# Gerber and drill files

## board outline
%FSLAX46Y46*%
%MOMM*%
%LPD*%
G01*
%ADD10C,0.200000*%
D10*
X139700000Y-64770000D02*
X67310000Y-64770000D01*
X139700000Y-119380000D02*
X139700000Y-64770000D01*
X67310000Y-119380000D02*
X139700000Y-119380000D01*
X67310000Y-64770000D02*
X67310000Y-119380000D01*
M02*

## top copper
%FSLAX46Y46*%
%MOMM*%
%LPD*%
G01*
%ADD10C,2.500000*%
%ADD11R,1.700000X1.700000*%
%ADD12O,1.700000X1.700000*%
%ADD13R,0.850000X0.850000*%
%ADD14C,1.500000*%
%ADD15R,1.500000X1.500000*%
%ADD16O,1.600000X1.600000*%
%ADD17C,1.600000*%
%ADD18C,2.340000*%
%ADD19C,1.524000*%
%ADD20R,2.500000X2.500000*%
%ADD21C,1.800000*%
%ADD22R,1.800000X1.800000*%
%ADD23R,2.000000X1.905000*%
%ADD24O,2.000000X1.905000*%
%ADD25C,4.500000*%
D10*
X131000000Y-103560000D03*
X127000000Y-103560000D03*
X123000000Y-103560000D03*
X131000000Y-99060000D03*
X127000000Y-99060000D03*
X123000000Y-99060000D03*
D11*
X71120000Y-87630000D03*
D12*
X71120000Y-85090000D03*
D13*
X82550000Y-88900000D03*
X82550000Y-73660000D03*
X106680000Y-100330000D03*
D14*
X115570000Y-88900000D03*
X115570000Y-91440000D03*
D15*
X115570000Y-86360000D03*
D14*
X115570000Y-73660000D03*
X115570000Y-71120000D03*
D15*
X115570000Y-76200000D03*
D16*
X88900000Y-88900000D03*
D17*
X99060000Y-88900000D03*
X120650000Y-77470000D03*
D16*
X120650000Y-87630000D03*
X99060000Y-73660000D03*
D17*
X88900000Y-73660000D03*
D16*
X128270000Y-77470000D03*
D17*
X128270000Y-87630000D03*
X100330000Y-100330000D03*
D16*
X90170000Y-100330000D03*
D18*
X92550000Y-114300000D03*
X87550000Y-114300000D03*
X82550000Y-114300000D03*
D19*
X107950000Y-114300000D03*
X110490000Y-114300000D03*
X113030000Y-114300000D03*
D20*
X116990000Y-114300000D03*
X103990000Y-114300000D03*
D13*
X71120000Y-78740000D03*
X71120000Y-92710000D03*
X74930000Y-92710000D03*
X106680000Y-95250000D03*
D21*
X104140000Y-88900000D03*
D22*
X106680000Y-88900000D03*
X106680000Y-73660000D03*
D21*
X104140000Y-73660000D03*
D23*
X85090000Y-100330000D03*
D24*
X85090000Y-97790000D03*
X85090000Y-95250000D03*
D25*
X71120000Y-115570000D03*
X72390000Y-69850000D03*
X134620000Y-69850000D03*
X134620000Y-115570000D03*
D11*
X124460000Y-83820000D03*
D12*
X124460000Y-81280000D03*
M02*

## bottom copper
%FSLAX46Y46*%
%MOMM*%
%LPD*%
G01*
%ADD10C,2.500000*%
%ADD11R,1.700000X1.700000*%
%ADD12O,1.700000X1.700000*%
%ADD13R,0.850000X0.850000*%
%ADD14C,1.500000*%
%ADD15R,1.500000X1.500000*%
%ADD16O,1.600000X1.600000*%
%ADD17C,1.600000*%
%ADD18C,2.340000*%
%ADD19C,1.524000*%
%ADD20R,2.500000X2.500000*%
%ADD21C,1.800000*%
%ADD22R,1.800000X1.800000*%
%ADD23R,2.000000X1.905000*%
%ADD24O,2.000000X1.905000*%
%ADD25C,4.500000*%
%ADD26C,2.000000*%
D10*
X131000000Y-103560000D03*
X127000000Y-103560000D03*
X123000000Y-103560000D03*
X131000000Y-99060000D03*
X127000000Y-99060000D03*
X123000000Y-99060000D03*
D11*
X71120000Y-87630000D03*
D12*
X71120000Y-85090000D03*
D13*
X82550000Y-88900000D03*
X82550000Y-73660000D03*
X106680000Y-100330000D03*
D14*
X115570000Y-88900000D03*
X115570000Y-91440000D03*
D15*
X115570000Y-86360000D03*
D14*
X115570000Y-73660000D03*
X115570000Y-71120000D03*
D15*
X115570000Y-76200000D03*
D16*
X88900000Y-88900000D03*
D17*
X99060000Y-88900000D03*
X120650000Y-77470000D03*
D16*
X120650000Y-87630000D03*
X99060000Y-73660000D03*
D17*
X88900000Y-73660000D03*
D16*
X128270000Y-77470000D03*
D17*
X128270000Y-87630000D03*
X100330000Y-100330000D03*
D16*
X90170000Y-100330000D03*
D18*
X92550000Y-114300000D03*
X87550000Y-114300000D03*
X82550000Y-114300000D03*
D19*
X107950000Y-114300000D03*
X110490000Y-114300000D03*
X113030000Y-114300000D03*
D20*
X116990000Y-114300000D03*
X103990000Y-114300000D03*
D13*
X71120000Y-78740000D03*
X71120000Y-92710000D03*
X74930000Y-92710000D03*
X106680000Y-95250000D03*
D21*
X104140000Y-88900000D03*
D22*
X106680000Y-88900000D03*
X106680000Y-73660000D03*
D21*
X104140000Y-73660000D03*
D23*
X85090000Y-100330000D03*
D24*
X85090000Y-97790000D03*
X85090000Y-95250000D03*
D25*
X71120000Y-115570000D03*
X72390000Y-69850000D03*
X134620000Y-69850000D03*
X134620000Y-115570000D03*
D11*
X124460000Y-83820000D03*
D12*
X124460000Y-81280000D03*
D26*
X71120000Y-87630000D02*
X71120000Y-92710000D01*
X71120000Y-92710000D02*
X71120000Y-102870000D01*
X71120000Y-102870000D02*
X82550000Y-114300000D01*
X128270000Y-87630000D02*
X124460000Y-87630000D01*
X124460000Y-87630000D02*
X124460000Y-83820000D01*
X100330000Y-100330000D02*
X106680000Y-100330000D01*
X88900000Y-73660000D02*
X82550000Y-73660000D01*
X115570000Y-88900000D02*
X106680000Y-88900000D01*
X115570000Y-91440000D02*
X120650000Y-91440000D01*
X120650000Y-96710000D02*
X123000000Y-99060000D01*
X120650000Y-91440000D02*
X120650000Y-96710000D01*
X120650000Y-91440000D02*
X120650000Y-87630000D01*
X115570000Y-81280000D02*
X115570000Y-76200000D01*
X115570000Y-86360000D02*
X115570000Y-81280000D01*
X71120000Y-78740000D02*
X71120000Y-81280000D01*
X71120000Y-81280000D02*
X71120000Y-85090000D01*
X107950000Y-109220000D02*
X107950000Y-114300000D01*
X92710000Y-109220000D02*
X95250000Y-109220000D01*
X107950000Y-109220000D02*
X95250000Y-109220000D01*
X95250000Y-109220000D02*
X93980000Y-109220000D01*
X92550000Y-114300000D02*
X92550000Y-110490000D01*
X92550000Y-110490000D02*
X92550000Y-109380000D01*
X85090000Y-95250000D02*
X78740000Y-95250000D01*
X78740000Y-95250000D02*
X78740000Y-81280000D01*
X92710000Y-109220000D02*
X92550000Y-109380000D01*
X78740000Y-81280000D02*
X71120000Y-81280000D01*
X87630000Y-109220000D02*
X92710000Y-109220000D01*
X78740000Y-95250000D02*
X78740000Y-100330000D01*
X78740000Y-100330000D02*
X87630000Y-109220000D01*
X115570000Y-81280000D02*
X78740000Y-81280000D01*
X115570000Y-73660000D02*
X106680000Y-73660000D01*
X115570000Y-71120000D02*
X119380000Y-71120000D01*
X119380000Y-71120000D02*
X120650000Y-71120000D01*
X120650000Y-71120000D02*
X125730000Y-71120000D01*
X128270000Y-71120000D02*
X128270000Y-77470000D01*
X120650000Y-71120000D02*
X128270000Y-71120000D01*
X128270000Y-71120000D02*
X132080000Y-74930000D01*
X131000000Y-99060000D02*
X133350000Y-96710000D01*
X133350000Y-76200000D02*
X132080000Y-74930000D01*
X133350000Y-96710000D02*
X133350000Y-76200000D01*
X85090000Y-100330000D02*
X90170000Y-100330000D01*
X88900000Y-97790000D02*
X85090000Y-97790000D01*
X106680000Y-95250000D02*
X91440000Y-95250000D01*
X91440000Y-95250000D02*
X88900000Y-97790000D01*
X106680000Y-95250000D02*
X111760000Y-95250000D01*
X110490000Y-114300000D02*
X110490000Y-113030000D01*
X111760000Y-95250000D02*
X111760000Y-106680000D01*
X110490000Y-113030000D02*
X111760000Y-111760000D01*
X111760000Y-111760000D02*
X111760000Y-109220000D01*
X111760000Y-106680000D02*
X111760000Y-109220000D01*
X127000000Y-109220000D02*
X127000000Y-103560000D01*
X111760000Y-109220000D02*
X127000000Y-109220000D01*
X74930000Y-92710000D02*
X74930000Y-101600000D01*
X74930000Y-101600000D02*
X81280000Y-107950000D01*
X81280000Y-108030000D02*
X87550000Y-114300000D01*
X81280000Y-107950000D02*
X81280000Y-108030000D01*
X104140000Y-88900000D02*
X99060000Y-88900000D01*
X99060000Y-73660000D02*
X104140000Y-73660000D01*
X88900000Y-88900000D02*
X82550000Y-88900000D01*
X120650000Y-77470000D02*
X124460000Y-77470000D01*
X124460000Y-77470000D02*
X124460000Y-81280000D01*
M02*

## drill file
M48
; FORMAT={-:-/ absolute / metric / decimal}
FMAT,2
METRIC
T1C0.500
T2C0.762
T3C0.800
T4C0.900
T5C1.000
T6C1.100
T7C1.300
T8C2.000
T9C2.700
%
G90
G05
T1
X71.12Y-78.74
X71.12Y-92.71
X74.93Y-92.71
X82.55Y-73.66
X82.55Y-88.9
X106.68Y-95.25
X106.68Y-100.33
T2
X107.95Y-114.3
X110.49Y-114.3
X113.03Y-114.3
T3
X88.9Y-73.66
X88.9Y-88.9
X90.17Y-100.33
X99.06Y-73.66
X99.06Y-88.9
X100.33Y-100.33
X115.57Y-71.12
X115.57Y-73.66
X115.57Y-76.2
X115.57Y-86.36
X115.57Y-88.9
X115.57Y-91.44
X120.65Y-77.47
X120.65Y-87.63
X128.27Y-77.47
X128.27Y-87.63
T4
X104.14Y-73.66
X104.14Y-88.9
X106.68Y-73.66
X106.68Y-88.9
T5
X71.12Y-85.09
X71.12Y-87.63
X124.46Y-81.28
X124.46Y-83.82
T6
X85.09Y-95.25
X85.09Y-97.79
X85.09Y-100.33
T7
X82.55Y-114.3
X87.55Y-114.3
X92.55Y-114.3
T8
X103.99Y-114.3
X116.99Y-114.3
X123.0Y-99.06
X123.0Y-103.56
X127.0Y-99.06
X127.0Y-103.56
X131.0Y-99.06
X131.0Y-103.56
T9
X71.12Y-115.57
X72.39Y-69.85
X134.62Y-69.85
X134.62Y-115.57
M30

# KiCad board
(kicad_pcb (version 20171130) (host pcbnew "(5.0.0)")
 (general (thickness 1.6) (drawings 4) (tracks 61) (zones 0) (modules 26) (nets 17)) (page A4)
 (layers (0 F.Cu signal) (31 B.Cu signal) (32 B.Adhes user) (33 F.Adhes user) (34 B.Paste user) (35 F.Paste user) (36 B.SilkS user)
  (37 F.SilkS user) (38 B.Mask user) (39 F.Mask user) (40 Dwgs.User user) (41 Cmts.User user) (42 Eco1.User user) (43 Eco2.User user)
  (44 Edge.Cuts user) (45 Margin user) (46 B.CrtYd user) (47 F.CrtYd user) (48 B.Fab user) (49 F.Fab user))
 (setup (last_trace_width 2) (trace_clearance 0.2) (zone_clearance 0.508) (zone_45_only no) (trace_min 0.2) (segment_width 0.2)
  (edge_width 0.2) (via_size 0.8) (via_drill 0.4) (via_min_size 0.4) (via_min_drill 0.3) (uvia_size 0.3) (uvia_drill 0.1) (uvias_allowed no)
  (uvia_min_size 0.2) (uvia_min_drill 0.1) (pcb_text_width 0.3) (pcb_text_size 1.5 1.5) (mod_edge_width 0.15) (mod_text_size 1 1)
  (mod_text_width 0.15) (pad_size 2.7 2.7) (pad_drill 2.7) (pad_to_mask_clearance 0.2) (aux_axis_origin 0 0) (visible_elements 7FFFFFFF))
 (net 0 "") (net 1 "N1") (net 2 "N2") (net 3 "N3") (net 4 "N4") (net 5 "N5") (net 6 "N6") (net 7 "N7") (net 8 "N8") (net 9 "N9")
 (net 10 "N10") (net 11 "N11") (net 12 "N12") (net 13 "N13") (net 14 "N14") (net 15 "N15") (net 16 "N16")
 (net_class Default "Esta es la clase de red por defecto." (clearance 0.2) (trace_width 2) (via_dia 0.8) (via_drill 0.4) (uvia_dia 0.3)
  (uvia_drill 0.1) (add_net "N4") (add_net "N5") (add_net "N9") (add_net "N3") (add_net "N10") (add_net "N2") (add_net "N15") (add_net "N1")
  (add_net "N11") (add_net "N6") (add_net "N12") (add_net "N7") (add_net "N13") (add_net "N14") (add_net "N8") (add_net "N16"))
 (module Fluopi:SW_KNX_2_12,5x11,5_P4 (layer F.Cu) (at 127 99.06)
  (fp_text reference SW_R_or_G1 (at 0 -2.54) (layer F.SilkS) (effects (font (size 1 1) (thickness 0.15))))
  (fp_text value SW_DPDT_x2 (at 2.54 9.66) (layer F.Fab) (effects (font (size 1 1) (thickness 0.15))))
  (pad 6 thru_hole circle (at 4 4.5) (size 2.5 2.5) (drill 2) (layers *.Cu *.Mask))
  (pad 2 thru_hole circle (at 0 4.5) (size 2.5 2.5) (drill 2) (layers *.Cu *.Mask) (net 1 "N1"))
  (pad 4 thru_hole circle (at -4 4.5) (size 2.5 2.5) (drill 2) (layers *.Cu *.Mask))
  (pad 3 thru_hole circle (at 4 0) (size 2.5 2.5) (drill 2) (layers *.Cu *.Mask) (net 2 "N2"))
  (pad 5 thru_hole circle (at 0 0) (size 2.5 2.5) (drill 2) (layers *.Cu *.Mask))
  (pad 1 thru_hole circle (at -4 0) (size 2.5 2.5) (drill 2) (layers *.Cu *.Mask) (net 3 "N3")))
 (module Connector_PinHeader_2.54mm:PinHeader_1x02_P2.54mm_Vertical (layer F.Cu) (at 71.12 87.63 180)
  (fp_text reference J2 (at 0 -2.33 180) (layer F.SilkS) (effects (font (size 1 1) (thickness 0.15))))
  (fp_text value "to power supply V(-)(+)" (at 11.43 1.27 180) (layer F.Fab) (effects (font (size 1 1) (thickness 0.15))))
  (pad 1 thru_hole rect (at 0 0 180) (size 1.7 1.7) (drill 1) (layers *.Cu *.Mask) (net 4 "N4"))
  (pad 2 thru_hole oval (at 0 2.54 180) (size 1.7 1.7) (drill 1) (layers *.Cu *.Mask) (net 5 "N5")))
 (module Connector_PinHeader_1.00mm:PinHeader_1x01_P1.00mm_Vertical (layer F.Cu) (at 82.55 88.9)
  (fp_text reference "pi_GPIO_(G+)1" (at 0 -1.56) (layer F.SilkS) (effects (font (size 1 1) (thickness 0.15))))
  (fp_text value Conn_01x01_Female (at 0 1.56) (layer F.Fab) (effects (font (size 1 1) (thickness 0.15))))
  (pad 1 thru_hole rect (at 0 0) (size 0.85 0.85) (drill 0.5) (layers *.Cu *.Mask) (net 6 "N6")))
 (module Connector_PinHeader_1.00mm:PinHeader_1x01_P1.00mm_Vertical (layer F.Cu) (at 82.55 73.66 180)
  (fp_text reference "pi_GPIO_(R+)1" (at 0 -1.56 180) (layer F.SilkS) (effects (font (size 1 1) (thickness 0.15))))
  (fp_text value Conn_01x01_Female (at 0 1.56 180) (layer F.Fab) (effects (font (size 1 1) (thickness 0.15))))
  (pad 1 thru_hole rect (at 0 0 180) (size 0.85 0.85) (drill 0.5) (layers *.Cu *.Mask) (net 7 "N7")))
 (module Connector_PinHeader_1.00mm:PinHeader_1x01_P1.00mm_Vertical (layer F.Cu) (at 106.68 100.33)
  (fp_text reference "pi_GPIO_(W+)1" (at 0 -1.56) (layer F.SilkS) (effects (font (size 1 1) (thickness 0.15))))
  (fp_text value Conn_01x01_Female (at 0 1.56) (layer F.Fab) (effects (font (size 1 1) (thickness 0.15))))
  (pad 1 thru_hole rect (at 0 0) (size 0.85 0.85) (drill 0.5) (layers *.Cu *.Mask) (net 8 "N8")))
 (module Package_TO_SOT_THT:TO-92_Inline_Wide (layer F.Cu) (at 115.57 86.36 270)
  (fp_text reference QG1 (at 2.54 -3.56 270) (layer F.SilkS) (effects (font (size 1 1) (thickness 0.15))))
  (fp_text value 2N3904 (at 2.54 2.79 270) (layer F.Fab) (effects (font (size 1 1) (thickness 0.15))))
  (pad 2 thru_hole circle (at 2.54 0) (size 1.5 1.5) (drill 0.8) (layers *.Cu *.Mask) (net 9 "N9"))
  (pad 3 thru_hole circle (at 5.08 0) (size 1.5 1.5) (drill 0.8) (layers *.Cu *.Mask) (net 3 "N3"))
  (pad 1 thru_hole rect (at 0 0) (size 1.5 1.5) (drill 0.8) (layers *.Cu *.Mask) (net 5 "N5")))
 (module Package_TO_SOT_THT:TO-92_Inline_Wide (layer F.Cu) (at 115.57 76.2 90)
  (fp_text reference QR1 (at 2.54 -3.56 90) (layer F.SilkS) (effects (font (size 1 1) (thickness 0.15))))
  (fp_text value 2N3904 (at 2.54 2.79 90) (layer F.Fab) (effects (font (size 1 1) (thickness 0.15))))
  (pad 2 thru_hole circle (at 2.54 0 180) (size 1.5 1.5) (drill 0.8) (layers *.Cu *.Mask) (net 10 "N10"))
  (pad 3 thru_hole circle (at 5.08 0 180) (size 1.5 1.5) (drill 0.8) (layers *.Cu *.Mask) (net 2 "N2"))
  (pad 1 thru_hole rect (at 0 0 180) (size 1.5 1.5) (drill 0.8) (layers *.Cu *.Mask) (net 5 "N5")))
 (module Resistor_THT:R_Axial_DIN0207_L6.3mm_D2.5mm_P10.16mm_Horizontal (layer F.Cu) (at 99.06 88.9 180)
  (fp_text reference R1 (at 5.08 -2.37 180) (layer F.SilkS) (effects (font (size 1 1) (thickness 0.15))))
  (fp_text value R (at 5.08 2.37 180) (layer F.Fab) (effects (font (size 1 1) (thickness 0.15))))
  (pad 2 thru_hole oval (at 10.16 0 180) (size 1.6 1.6) (drill 0.8) (layers *.Cu *.Mask) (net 6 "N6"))
  (pad 1 thru_hole circle (at 0 0 180) (size 1.6 1.6) (drill 0.8) (layers *.Cu *.Mask) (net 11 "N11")))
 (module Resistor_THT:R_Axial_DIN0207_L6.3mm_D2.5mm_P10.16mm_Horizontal (layer F.Cu) (at 120.65 77.47 270)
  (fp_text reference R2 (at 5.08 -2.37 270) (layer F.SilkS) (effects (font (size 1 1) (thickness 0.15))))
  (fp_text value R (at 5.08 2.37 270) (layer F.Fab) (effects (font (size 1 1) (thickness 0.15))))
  (pad 1 thru_hole circle (at 0 0 270) (size 1.6 1.6) (drill 0.8) (layers *.Cu *.Mask) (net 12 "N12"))
  (pad 2 thru_hole oval (at 10.16 0 270) (size 1.6 1.6) (drill 0.8) (layers *.Cu *.Mask) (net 3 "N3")))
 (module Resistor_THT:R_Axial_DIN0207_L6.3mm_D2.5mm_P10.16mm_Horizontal (layer F.Cu) (at 88.9 73.66)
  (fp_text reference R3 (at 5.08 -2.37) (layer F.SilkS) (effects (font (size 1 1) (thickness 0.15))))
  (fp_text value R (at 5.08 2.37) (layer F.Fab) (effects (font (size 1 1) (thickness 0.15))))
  (pad 2 thru_hole oval (at 10.16 0) (size 1.6 1.6) (drill 0.8) (layers *.Cu *.Mask) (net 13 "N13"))
  (pad 1 thru_hole circle (at 0 0) (size 1.6 1.6) (drill 0.8) (layers *.Cu *.Mask) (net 7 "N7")))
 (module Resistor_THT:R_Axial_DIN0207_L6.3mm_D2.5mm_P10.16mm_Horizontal (layer F.Cu) (at 128.27 87.63 90)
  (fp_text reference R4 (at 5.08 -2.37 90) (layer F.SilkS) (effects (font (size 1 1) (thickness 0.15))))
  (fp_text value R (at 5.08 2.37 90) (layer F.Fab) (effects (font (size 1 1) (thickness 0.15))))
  (pad 2 thru_hole oval (at 10.16 0 90) (size 1.6 1.6) (drill 0.8) (layers *.Cu *.Mask) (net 2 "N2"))
  (pad 1 thru_hole circle (at 0 0 90) (size 1.6 1.6) (drill 0.8) (layers *.Cu *.Mask) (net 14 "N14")))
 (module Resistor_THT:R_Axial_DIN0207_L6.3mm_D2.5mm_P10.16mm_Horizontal (layer F.Cu) (at 100.33 100.33 180)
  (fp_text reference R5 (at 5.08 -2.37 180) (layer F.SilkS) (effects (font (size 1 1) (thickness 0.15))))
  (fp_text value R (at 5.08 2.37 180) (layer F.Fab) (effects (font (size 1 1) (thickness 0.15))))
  (pad 1 thru_hole circle (at 0 0 180) (size 1.6 1.6) (drill 0.8) (layers *.Cu *.Mask) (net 8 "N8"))
  (pad 2 thru_hole oval (at 10.16 0 180) (size 1.6 1.6) (drill 0.8) (layers *.Cu *.Mask) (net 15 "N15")))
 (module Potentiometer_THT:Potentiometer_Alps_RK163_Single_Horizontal (layer F.Cu) (at 82.55 114.3 270)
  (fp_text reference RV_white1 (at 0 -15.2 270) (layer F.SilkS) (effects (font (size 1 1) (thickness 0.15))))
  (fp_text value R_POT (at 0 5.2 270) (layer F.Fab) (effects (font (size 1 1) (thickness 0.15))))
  (pad 3 thru_hole circle (at 0 -10 270) (size 2.34 2.34) (drill 1.3) (layers *.Cu *.Mask) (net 5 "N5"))
  (pad 2 thru_hole circle (at 0 -5 270) (size 2.34 2.34) (drill 1.3) (layers *.Cu *.Mask) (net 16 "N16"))
  (pad 1 thru_hole circle (at 0 0 270) (size 2.34 2.34) (drill 1.3) (layers *.Cu *.Mask) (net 4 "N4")))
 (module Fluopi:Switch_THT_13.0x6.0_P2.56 (layer F.Cu) (at 110.49 114.3)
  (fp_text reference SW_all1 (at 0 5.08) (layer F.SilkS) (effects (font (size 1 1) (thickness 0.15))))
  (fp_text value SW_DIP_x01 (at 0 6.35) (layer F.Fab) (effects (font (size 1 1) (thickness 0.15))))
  (pad 1 thru_hole circle (at -2.54 0) (size 1.524 1.524) (drill 0.762) (layers *.Cu *.Mask) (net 5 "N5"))
  (pad 2 thru_hole circle (at 0 0) (size 1.524 1.524) (drill 0.762) (layers *.Cu *.Mask) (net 1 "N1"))
  (pad 3 thru_hole circle (at 2.54 0) (size 1.524 1.524) (drill 0.762) (layers *.Cu *.Mask))
  (pad 4 thru_hole rect (at 6.5 0) (size 2.5 2.5) (drill 2) (layers *.Cu *.Mask))
  (pad 4 thru_hole rect (at -6.5 0) (size 2.5 2.5) (drill 2) (layers *.Cu *.Mask)))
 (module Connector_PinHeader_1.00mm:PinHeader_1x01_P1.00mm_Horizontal (layer F.Cu) (at 71.12 78.74 180)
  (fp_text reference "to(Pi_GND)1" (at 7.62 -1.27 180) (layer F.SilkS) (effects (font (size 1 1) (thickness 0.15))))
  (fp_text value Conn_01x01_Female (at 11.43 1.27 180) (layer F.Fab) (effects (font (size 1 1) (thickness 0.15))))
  (pad 1 thru_hole rect (at 0 0 180) (size 0.85 0.85) (drill 0.5) (layers *.Cu *.Mask) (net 5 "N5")))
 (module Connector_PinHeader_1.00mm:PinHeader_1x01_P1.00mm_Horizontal (layer F.Cu) (at 71.12 92.71 180)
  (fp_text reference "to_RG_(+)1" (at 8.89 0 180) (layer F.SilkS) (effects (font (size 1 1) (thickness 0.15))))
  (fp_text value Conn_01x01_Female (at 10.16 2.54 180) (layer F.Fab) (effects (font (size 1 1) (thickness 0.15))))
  (pad 1 thru_hole rect (at 0 0 180) (size 0.85 0.85) (drill 0.5) (layers *.Cu *.Mask) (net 4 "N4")))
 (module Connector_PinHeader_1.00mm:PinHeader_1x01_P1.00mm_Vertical (layer F.Cu) (at 74.93 92.71)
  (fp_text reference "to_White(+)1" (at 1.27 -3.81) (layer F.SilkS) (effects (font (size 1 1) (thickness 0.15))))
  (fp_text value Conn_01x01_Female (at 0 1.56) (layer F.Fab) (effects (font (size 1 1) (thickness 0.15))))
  (pad 1 thru_hole rect (at 0 0) (size 0.85 0.85) (drill 0.5) (layers *.Cu *.Mask) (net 16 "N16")))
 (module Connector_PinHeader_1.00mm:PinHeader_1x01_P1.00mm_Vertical (layer F.Cu) (at 106.68 95.25)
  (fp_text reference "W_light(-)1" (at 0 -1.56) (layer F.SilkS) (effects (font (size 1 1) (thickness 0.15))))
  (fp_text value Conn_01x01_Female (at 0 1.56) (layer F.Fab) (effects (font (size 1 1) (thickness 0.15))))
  (pad 1 thru_hole rect (at 0 0) (size 0.85 0.85) (drill 0.5) (layers *.Cu *.Mask) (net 1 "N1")))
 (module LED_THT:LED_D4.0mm (layer F.Cu) (at 106.68 88.9 180)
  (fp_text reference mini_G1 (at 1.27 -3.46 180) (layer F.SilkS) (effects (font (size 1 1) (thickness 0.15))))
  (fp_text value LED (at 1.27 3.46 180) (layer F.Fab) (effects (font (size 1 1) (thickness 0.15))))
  (pad 2 thru_hole circle (at 2.54 0 180) (size 1.8 1.8) (drill 0.9) (layers *.Cu *.Mask) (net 11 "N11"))
  (pad 1 thru_hole rect (at 0 0 180) (size 1.8 1.8) (drill 0.9) (layers *.Cu *.Mask) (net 9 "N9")))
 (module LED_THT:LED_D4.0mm (layer F.Cu) (at 106.68 73.66 180)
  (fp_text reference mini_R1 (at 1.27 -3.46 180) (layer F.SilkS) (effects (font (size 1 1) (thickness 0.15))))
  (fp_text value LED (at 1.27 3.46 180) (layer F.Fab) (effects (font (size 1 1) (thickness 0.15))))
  (pad 1 thru_hole rect (at 0 0 180) (size 1.8 1.8) (drill 0.9) (layers *.Cu *.Mask) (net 10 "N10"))
  (pad 2 thru_hole circle (at 2.54 0 180) (size 1.8 1.8) (drill 0.9) (layers *.Cu *.Mask) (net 13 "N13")))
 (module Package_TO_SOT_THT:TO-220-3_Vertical (layer F.Cu) (at 85.09 100.33 90)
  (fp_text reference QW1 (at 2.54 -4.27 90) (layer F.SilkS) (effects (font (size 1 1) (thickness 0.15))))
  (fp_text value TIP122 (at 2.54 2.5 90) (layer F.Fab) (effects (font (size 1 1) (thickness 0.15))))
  (pad 1 thru_hole rect (at 0 0 90) (size 1.905 2) (drill 1.1) (layers *.Cu *.Mask) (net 15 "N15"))
  (pad 2 thru_hole oval (at 2.54 0 90) (size 1.905 2) (drill 1.1) (layers *.Cu *.Mask) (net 1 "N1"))
  (pad 3 thru_hole oval (at 5.08 0 90) (size 1.905 2) (drill 1.1) (layers *.Cu *.Mask) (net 5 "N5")))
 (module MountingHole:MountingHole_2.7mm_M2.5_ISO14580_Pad (layer F.Cu) (at 71.12 115.57)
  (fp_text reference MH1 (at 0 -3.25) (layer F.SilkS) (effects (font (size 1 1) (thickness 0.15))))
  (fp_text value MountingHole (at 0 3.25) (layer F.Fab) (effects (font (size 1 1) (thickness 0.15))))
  (pad 1 thru_hole circle (at 0 0) (size 4.5 4.5) (drill 2.7) (layers *.Cu *.Mask)))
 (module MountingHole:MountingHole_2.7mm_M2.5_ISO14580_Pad (layer F.Cu) (at 72.39 69.85)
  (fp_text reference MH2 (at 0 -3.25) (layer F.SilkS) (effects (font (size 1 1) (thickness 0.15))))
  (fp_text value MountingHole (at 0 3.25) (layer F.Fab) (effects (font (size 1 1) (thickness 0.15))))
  (pad 1 thru_hole circle (at 0 0) (size 4.5 4.5) (drill 2.7) (layers *.Cu *.Mask)))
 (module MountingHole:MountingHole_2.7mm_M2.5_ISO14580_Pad (layer F.Cu) (at 134.62 69.85)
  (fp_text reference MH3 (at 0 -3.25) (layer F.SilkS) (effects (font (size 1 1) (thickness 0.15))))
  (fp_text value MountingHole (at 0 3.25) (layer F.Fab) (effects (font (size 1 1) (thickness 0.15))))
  (pad 1 thru_hole circle (at 0 0) (size 4.5 4.5) (drill 2.7) (layers *.Cu *.Mask)))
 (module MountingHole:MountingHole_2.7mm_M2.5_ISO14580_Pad (layer F.Cu) (at 134.62 115.57)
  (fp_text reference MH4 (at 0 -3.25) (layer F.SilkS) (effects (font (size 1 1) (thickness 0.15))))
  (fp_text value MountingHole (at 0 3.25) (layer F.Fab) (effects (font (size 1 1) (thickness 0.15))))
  (pad 1 thru_hole circle (at 0 0) (size 4.5 4.5) (drill 2.7) (layers *.Cu *.Mask)))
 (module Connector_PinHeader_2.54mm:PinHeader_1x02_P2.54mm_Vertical (layer F.Cu) (at 124.46 83.82 180)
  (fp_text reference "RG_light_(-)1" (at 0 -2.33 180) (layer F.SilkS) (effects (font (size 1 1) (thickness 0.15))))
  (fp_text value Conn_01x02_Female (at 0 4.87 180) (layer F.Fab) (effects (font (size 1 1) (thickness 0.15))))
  (pad 1 thru_hole rect (at 0 0 180) (size 1.7 1.7) (drill 1) (layers *.Cu *.Mask) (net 14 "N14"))
  (pad 2 thru_hole oval (at 0 2.54 180) (size 1.7 1.7) (drill 1) (layers *.Cu *.Mask) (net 12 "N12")))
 (gr_line (start 139.7 64.77) (end 67.31 64.77) (layer Edge.Cuts) (width 0.2))
 (gr_line (start 139.7 119.38) (end 139.7 64.77) (layer Edge.Cuts) (width 0.2))
 (gr_line (start 67.31 119.38) (end 139.7 119.38) (layer Edge.Cuts) (width 0.2))
 (gr_line (start 67.31 64.77) (end 67.31 119.38) (layer Edge.Cuts) (width 0.2))
 (segment (start 71.12 87.63) (end 71.12 92.71) (width 2) (layer B.Cu) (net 4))
 (segment (start 71.12 92.71) (end 71.12 102.87) (width 2) (layer B.Cu) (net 4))
 (segment (start 71.12 102.87) (end 82.55 114.3) (width 2) (layer B.Cu) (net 4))
 (segment (start 128.27 87.63) (end 124.46 87.63) (width 2) (layer B.Cu) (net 14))
 (segment (start 124.46 87.63) (end 124.46 83.82) (width 2) (layer B.Cu) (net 14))
 (segment (start 100.33 100.33) (end 106.68 100.33) (width 2) (layer B.Cu) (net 8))
 (segment (start 88.9 73.66) (end 82.55 73.66) (width 2) (layer B.Cu) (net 7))
 (segment (start 115.57 88.9) (end 106.68 88.9) (width 2) (layer B.Cu) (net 9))
 (segment (start 115.57 91.44) (end 120.65 91.44) (width 2) (layer B.Cu) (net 3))
 (segment (start 120.65 96.71) (end 123 99.06) (width 2) (layer B.Cu) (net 3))
 (segment (start 120.65 91.44) (end 120.65 96.71) (width 2) (layer B.Cu) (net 3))
 (segment (start 120.65 91.44) (end 120.65 87.63) (width 2) (layer B.Cu) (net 3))
 (segment (start 115.57 81.28) (end 115.57 76.2) (width 2) (layer B.Cu) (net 5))
 (segment (start 115.57 86.36) (end 115.57 81.28) (width 2) (layer B.Cu) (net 5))
 (segment (start 71.12 78.74) (end 71.12 81.28) (width 2) (layer B.Cu) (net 5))
 (segment (start 71.12 81.28) (end 71.12 85.09) (width 2) (layer B.Cu) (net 5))
 (segment (start 107.95 109.22) (end 107.95 114.3) (width 2) (layer B.Cu) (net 5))
 (segment (start 92.71 109.22) (end 95.25 109.22) (width 2) (layer B.Cu) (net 5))
 (segment (start 107.95 109.22) (end 95.25 109.22) (width 2) (layer B.Cu) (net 5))
 (segment (start 95.25 109.22) (end 93.98 109.22) (width 2) (layer B.Cu) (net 5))
 (segment (start 92.55 114.3) (end 92.55 110.49) (width 2) (layer B.Cu) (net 5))
 (segment (start 92.55 110.49) (end 92.55 109.38) (width 2) (layer B.Cu) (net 5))
 (segment (start 85.09 95.25) (end 78.74 95.25) (width 2) (layer B.Cu) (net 5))
 (segment (start 78.74 95.25) (end 78.74 81.28) (width 2) (layer B.Cu) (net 5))
 (segment (start 92.71 109.22) (end 92.55 109.38) (width 2) (layer B.Cu) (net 5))
 (segment (start 78.74 81.28) (end 71.12 81.28) (width 2) (layer B.Cu) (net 5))
 (segment (start 87.63 109.22) (end 92.71 109.22) (width 2) (layer B.Cu) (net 5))
 (segment (start 78.74 95.25) (end 78.74 100.33) (width 2) (layer B.Cu) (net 5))
 (segment (start 78.74 100.33) (end 87.63 109.22) (width 2) (layer B.Cu) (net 5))
 (segment (start 115.57 81.28) (end 78.74 81.28) (width 2) (layer B.Cu) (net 5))
 (segment (start 115.57 73.66) (end 106.68 73.66) (width 2) (layer B.Cu) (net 10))
 (segment (start 115.57 71.12) (end 119.38 71.12) (width 2) (layer B.Cu) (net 2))
 (segment (start 119.38 71.12) (end 120.65 71.12) (width 2) (layer B.Cu) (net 2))
 (segment (start 120.65 71.12) (end 125.73 71.12) (width 2) (layer B.Cu) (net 2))
 (segment (start 128.27 71.12) (end 128.27 77.47) (width 2) (layer B.Cu) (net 2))
 (segment (start 120.65 71.12) (end 128.27 71.12) (width 2) (layer B.Cu) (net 2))
 (segment (start 128.27 71.12) (end 132.08 74.93) (width 2) (layer B.Cu) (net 2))
 (segment (start 131 99.06) (end 133.35 96.71) (width 2) (layer B.Cu) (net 2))
 (segment (start 133.35 76.2) (end 132.08 74.93) (width 2) (layer B.Cu) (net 2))
 (segment (start 133.35 96.71) (end 133.35 76.2) (width 2) (layer B.Cu) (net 2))
 (segment (start 85.09 100.33) (end 90.17 100.33) (width 2) (layer B.Cu) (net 15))
 (segment (start 88.9 97.79) (end 85.09 97.79) (width 2) (layer B.Cu) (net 1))
 (segment (start 106.68 95.25) (end 91.44 95.25) (width 2) (layer B.Cu) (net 1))
 (segment (start 91.44 95.25) (end 88.9 97.79) (width 2) (layer B.Cu) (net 1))
 (segment (start 106.68 95.25) (end 111.76 95.25) (width 2) (layer B.Cu) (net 1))
 (segment (start 110.49 114.3) (end 110.49 113.03) (width 2) (layer B.Cu) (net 1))
 (segment (start 111.76 95.25) (end 111.76 106.68) (width 2) (layer B.Cu) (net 1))
 (segment (start 110.49 113.03) (end 111.76 111.76) (width 2) (layer B.Cu) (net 1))
 (segment (start 111.76 111.76) (end 111.76 109.22) (width 2) (layer B.Cu) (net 1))
 (segment (start 111.76 106.68) (end 111.76 109.22) (width 2) (layer B.Cu) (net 1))
 (segment (start 127 109.22) (end 127 103.56) (width 2) (layer B.Cu) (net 1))
 (segment (start 111.76 109.22) (end 127 109.22) (width 2) (layer B.Cu) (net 1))
 (segment (start 74.93 92.71) (end 74.93 101.6) (width 2) (layer B.Cu) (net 16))
 (segment (start 74.93 101.6) (end 81.28 107.95) (width 2) (layer B.Cu) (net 16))
 (segment (start 81.28 108.03) (end 87.55 114.3) (width 2) (layer B.Cu) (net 16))
 (segment (start 81.28 107.95) (end 81.28 108.03) (width 2) (layer B.Cu) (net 16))
 (segment (start 104.14 88.9) (end 99.06 88.9) (width 2) (layer B.Cu) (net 11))
 (segment (start 99.06 73.66) (end 104.14 73.66) (width 2) (layer B.Cu) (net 13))
 (segment (start 88.9 88.9) (end 82.55 88.9) (width 2) (layer B.Cu) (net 6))
 (segment (start 120.65 77.47) (end 124.46 77.47) (width 2) (layer B.Cu) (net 12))
 (segment (start 124.46 77.47) (end 124.46 81.28) (width 2) (layer B.Cu) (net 12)))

